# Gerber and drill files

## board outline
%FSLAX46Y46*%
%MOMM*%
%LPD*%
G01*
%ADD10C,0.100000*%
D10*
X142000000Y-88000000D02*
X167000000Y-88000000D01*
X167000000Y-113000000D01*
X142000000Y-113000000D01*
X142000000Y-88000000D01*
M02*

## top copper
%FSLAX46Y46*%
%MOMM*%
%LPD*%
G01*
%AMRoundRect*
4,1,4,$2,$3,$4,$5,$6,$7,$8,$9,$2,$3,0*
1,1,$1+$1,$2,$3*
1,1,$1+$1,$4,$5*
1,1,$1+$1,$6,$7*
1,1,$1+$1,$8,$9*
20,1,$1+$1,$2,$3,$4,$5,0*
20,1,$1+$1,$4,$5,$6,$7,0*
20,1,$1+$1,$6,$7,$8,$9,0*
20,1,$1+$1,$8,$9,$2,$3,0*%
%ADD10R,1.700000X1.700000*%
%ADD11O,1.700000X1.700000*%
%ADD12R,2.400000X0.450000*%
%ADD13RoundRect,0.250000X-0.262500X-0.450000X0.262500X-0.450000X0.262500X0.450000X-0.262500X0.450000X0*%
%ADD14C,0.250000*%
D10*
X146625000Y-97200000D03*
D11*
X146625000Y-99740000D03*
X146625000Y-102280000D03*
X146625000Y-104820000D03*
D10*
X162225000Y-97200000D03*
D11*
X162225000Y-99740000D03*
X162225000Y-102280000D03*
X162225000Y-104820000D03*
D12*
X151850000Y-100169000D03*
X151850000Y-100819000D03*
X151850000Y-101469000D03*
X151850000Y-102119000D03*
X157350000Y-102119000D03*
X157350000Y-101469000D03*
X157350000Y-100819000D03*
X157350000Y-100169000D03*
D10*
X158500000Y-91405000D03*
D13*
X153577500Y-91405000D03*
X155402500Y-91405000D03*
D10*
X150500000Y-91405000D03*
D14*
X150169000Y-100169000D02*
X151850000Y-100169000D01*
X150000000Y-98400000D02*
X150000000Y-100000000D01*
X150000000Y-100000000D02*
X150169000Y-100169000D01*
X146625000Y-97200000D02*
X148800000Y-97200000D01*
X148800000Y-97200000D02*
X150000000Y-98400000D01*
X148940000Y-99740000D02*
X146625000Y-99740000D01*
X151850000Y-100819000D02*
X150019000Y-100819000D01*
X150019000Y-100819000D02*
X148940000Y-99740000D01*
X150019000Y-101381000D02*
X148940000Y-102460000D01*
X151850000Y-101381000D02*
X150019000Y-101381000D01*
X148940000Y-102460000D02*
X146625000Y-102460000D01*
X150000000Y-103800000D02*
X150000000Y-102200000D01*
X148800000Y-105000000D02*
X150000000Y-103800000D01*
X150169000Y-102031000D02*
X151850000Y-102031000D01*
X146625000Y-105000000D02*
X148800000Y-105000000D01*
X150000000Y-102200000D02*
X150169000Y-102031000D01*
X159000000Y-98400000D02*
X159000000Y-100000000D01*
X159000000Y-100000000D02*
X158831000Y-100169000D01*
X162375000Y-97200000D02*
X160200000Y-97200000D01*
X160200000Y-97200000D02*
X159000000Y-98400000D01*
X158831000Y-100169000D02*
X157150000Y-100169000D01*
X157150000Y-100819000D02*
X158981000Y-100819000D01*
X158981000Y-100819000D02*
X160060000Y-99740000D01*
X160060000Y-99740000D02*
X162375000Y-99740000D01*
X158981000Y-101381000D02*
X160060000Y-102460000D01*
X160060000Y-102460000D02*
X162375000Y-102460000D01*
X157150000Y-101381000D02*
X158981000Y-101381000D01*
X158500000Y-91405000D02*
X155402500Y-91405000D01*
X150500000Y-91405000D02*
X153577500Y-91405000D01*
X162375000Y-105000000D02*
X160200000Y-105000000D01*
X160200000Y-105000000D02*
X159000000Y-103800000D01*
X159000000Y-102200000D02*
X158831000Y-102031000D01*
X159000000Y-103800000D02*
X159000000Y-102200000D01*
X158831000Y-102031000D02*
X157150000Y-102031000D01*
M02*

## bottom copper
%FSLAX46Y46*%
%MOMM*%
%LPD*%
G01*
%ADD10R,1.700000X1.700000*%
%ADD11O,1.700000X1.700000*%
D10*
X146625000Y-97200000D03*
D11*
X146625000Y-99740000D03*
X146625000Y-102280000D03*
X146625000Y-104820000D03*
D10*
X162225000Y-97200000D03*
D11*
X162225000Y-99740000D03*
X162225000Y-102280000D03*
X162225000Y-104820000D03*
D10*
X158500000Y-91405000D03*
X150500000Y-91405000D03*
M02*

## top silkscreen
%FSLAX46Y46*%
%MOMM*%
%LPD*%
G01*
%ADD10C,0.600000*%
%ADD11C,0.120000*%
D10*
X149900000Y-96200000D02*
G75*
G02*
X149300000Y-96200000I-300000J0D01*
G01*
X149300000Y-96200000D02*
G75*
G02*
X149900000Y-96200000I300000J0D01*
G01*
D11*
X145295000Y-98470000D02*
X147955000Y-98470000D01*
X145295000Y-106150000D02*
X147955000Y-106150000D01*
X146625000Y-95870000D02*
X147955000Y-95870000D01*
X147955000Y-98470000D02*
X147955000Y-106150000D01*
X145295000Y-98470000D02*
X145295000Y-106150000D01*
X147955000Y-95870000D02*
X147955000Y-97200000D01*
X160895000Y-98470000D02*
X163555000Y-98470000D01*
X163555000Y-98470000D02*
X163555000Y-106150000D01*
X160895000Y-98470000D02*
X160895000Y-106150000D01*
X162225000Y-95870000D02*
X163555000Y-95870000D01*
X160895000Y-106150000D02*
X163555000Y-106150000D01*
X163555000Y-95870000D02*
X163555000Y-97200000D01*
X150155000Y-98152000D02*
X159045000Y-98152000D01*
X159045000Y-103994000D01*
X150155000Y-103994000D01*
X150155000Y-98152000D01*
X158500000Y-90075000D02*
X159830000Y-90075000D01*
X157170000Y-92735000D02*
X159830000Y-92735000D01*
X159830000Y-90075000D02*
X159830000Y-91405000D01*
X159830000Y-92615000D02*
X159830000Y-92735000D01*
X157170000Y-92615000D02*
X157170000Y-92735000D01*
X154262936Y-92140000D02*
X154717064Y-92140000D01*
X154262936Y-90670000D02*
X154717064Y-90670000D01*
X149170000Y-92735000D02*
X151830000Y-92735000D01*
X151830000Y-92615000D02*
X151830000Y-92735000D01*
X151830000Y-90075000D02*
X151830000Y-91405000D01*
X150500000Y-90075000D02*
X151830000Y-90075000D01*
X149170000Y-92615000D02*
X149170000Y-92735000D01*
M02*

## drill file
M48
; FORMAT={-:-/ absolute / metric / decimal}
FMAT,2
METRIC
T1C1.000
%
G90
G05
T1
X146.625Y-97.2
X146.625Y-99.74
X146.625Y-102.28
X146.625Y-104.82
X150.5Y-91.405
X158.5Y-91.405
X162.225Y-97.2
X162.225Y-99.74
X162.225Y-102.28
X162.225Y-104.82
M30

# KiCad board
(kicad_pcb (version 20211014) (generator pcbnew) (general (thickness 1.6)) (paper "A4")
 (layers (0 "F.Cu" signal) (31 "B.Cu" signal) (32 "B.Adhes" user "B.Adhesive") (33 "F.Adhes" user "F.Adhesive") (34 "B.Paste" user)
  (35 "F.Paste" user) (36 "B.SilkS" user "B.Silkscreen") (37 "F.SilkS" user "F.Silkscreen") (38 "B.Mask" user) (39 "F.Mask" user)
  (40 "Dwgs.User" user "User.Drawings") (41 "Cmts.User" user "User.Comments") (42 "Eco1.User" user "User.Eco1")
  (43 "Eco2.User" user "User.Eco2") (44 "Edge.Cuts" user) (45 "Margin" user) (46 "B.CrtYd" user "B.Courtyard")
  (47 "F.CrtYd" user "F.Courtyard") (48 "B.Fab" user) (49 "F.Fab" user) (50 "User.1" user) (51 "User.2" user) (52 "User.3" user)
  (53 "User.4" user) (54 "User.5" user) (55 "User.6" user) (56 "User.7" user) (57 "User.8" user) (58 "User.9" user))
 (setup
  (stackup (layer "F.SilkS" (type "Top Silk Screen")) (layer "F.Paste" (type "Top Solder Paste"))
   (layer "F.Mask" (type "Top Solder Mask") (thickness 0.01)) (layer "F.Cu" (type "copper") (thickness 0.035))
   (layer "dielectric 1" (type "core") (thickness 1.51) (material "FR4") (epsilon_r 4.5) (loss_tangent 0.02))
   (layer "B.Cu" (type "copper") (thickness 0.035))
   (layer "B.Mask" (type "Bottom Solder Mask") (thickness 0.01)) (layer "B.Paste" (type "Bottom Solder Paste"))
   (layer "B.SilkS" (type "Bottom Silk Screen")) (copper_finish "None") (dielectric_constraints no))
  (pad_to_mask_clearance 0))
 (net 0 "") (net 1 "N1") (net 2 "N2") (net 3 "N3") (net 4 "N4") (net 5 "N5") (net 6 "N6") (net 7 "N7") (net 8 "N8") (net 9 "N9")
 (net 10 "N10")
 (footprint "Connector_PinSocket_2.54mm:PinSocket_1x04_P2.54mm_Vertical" (layer "F.Cu") (at 146.625 97.2)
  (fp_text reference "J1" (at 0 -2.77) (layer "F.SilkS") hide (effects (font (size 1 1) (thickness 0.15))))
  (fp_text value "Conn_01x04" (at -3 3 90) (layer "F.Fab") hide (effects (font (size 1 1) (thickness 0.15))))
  (fp_line (start -1.33 1.27) (end 1.33 1.27) (layer "F.SilkS") (width 0.12))
  (fp_line (start -1.33 8.95) (end 1.33 8.95) (layer "F.SilkS") (width 0.12))
  (fp_line (start 0 -1.33) (end 1.33 -1.33) (layer "F.SilkS") (width 0.12))
  (fp_line (start 1.33 1.27) (end 1.33 8.95) (layer "F.SilkS") (width 0.12))
  (fp_line (start -1.33 1.27) (end -1.33 8.95) (layer "F.SilkS") (width 0.12))
  (fp_line (start 1.33 -1.33) (end 1.33 0) (layer "F.SilkS") (width 0.12))
  (pad "1" thru_hole rect (at 0 0) (size 1.7 1.7) (drill 1) (layers *.Cu *.Mask) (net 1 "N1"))
  (pad "2" thru_hole oval (at 0 2.54) (size 1.7 1.7) (drill 1) (layers *.Cu *.Mask) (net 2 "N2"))
  (pad "3" thru_hole oval (at 0 5.08) (size 1.7 1.7) (drill 1) (layers *.Cu *.Mask) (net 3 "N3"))
  (pad "4" thru_hole oval (at 0 7.62) (size 1.7 1.7) (drill 1) (layers *.Cu *.Mask) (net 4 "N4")))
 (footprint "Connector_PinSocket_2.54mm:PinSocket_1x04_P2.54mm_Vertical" (layer "F.Cu") (at 162.225 97.2)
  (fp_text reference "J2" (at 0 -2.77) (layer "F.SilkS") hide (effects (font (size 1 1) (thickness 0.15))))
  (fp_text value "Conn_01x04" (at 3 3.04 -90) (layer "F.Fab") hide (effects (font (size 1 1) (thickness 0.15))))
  (fp_line (start -1.33 1.27) (end 1.33 1.27) (layer "F.SilkS") (width 0.12))
  (fp_line (start 1.33 1.27) (end 1.33 8.95) (layer "F.SilkS") (width 0.12))
  (fp_line (start -1.33 1.27) (end -1.33 8.95) (layer "F.SilkS") (width 0.12))
  (fp_line (start 0 -1.33) (end 1.33 -1.33) (layer "F.SilkS") (width 0.12))
  (fp_line (start -1.33 8.95) (end 1.33 8.95) (layer "F.SilkS") (width 0.12))
  (fp_line (start 1.33 -1.33) (end 1.33 0) (layer "F.SilkS") (width 0.12))
  (pad "1" thru_hole rect (at 0 0) (size 1.7 1.7) (drill 1) (layers *.Cu *.Mask) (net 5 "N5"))
  (pad "2" thru_hole oval (at 0 2.54) (size 1.7 1.7) (drill 1) (layers *.Cu *.Mask) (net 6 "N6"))
  (pad "3" thru_hole oval (at 0 5.08) (size 1.7 1.7) (drill 1) (layers *.Cu *.Mask) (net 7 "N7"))
  (pad "4" thru_hole oval (at 0 7.62) (size 1.7 1.7) (drill 1) (layers *.Cu *.Mask) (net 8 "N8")))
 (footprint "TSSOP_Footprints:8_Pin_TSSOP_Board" (layer "F.Cu") (at 154.6 101.2)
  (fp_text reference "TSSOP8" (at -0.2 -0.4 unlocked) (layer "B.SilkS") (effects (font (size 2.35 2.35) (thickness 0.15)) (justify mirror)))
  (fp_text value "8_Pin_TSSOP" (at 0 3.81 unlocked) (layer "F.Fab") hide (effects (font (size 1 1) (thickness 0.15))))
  (fp_rect (start -4.445 -3.048) (end 4.445 2.794) (layer "F.SilkS") (width 0.12) (fill none))
  (pad "1" smd rect (at -2.75 -1.031) (size 2.4 0.45) (layers "F.Cu" "F.Paste" "F.Mask") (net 1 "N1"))
  (pad "2" smd rect (at -2.75 -0.381) (size 2.4 0.45) (layers "F.Cu" "F.Paste" "F.Mask") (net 2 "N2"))
  (pad "3" smd rect (at -2.75 0.269) (size 2.4 0.45) (layers "F.Cu" "F.Paste" "F.Mask") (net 3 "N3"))
  (pad "4" smd rect (at -2.75 0.919) (size 2.4 0.45) (layers "F.Cu" "F.Paste" "F.Mask") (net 4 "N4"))
  (pad "5" smd rect (at 2.75 0.919) (size 2.4 0.45) (layers "F.Cu" "F.Paste" "F.Mask") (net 8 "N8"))
  (pad "6" smd rect (at 2.75 0.269) (size 2.4 0.45) (layers "F.Cu" "F.Paste" "F.Mask") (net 7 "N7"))
  (pad "7" smd rect (at 2.75 -0.381) (size 2.4 0.45) (layers "F.Cu" "F.Paste" "F.Mask") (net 6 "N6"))
  (pad "8" smd rect (at 2.75 -1.031) (size 2.4 0.45) (layers "F.Cu" "F.Paste" "F.Mask") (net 5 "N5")))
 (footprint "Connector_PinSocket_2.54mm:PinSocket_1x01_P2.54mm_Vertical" (layer "F.Cu") (at 158.5 91.405)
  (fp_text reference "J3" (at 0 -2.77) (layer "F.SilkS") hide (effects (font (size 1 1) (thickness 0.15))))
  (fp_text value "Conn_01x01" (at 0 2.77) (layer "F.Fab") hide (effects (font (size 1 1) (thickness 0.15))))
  (fp_line (start 0 -1.33) (end 1.33 -1.33) (layer "F.SilkS") (width 0.12))
  (fp_line (start -1.33 1.33) (end 1.33 1.33) (layer "F.SilkS") (width 0.12))
  (fp_line (start 1.33 -1.33) (end 1.33 0) (layer "F.SilkS") (width 0.12))
  (fp_line (start 1.33 1.21) (end 1.33 1.33) (layer "F.SilkS") (width 0.12))
  (fp_line (start -1.33 1.21) (end -1.33 1.33) (layer "F.SilkS") (width 0.12))
  (pad "1" thru_hole rect (at 0 0) (size 1.7 1.7) (drill 1) (layers *.Cu *.Mask) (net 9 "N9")))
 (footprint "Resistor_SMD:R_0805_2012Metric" (layer "F.Cu") (at 154.49 91.405)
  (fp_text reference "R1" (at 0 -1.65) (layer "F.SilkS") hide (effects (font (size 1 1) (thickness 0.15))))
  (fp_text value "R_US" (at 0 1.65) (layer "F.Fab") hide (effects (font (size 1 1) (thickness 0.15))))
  (fp_line (start -0.227064 0.735) (end 0.227064 0.735) (layer "F.SilkS") (width 0.12))
  (fp_line (start -0.227064 -0.735) (end 0.227064 -0.735) (layer "F.SilkS") (width 0.12))
  (pad "1" smd roundrect (at -0.9125 0) (size 1.025 1.4) (layers "F.Cu" "F.Paste" "F.Mask") (roundrect_rratio 0.243902) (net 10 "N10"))
  (pad "2" smd roundrect (at 0.9125 0) (size 1.025 1.4) (layers "F.Cu" "F.Paste" "F.Mask") (roundrect_rratio 0.243902) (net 9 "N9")))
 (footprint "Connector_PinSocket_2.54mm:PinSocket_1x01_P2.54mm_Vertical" (layer "F.Cu") (at 150.5 91.405)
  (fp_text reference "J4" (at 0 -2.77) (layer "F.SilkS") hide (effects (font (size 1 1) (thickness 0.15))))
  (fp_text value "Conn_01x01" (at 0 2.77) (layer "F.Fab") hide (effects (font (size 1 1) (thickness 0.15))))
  (fp_line (start -1.33 1.33) (end 1.33 1.33) (layer "F.SilkS") (width 0.12))
  (fp_line (start 1.33 1.21) (end 1.33 1.33) (layer "F.SilkS") (width 0.12))
  (fp_line (start 1.33 -1.33) (end 1.33 0) (layer "F.SilkS") (width 0.12))
  (fp_line (start 0 -1.33) (end 1.33 -1.33) (layer "F.SilkS") (width 0.12))
  (fp_line (start -1.33 1.21) (end -1.33 1.33) (layer "F.SilkS") (width 0.12))
  (pad "1" thru_hole rect (at 0 0) (size 1.7 1.7) (drill 1) (layers *.Cu *.Mask) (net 10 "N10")))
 (gr_circle (center 149.6 96.2) (end 150.1 96.2) (layer "F.SilkS") (width 0.2) (fill solid))
 (gr_rect (start 142 88) (end 167 113) (layer "Edge.Cuts") (width 0.1) (fill none))
 (segment (start 150.169 100.169) (end 151.85 100.169) (width 0.25) (layer "F.Cu") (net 1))
 (segment (start 150 98.4) (end 150 100) (width 0.25) (layer "F.Cu") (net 1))
 (segment (start 150 100) (end 150.169 100.169) (width 0.25) (layer "F.Cu") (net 1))
 (segment (start 146.625 97.2) (end 148.8 97.2) (width 0.25) (layer "F.Cu") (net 1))
 (segment (start 148.8 97.2) (end 150 98.4) (width 0.25) (layer "F.Cu") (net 1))
 (segment (start 148.94 99.74) (end 146.625 99.74) (width 0.25) (layer "F.Cu") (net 2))
 (segment (start 151.85 100.819) (end 150.019 100.819) (width 0.25) (layer "F.Cu") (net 2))
 (segment (start 150.019 100.819) (end 148.94 99.74) (width 0.25) (layer "F.Cu") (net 2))
 (segment (start 150.019 101.381) (end 148.94 102.46) (width 0.25) (layer "F.Cu") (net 3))
 (segment (start 151.85 101.381) (end 150.019 101.381) (width 0.25) (layer "F.Cu") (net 3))
 (segment (start 148.94 102.46) (end 146.625 102.46) (width 0.25) (layer "F.Cu") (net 3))
 (segment (start 150 103.8) (end 150 102.2) (width 0.25) (layer "F.Cu") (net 4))
 (segment (start 148.8 105) (end 150 103.8) (width 0.25) (layer "F.Cu") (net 4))
 (segment (start 150.169 102.031) (end 151.85 102.031) (width 0.25) (layer "F.Cu") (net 4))
 (segment (start 146.625 105) (end 148.8 105) (width 0.25) (layer "F.Cu") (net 4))
 (segment (start 150 102.2) (end 150.169 102.031) (width 0.25) (layer "F.Cu") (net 4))
 (segment (start 159 98.4) (end 159 100) (width 0.25) (layer "F.Cu") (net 5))
 (segment (start 159 100) (end 158.831 100.169) (width 0.25) (layer "F.Cu") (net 5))
 (segment (start 162.375 97.2) (end 160.2 97.2) (width 0.25) (layer "F.Cu") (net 5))
 (segment (start 160.2 97.2) (end 159 98.4) (width 0.25) (layer "F.Cu") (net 5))
 (segment (start 158.831 100.169) (end 157.15 100.169) (width 0.25) (layer "F.Cu") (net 5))
 (segment (start 157.15 100.819) (end 158.981 100.819) (width 0.25) (layer "F.Cu") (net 6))
 (segment (start 158.981 100.819) (end 160.06 99.74) (width 0.25) (layer "F.Cu") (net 6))
 (segment (start 160.06 99.74) (end 162.375 99.74) (width 0.25) (layer "F.Cu") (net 6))
 (segment (start 158.981 101.381) (end 160.06 102.46) (width 0.25) (layer "F.Cu") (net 7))
 (segment (start 160.06 102.46) (end 162.375 102.46) (width 0.25) (layer "F.Cu") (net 7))
 (segment (start 157.15 101.381) (end 158.981 101.381) (width 0.25) (layer "F.Cu") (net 7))
 (segment (start 158.5 91.405) (end 155.4025 91.405) (width 0.25) (layer "F.Cu") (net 9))
 (segment (start 150.5 91.405) (end 153.5775 91.405) (width 0.25) (layer "F.Cu") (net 10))
 (segment (start 162.375 105) (end 160.2 105) (width 0.25) (layer "F.Cu") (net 8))
 (segment (start 160.2 105) (end 159 103.8) (width 0.25) (layer "F.Cu") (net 8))
 (segment (start 159 102.2) (end 158.831 102.031) (width 0.25) (layer "F.Cu") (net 8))
 (segment (start 159 103.8) (end 159 102.2) (width 0.25) (layer "F.Cu") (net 8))
 (segment (start 158.831 102.031) (end 157.15 102.031) (width 0.25) (layer "F.Cu") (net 8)))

